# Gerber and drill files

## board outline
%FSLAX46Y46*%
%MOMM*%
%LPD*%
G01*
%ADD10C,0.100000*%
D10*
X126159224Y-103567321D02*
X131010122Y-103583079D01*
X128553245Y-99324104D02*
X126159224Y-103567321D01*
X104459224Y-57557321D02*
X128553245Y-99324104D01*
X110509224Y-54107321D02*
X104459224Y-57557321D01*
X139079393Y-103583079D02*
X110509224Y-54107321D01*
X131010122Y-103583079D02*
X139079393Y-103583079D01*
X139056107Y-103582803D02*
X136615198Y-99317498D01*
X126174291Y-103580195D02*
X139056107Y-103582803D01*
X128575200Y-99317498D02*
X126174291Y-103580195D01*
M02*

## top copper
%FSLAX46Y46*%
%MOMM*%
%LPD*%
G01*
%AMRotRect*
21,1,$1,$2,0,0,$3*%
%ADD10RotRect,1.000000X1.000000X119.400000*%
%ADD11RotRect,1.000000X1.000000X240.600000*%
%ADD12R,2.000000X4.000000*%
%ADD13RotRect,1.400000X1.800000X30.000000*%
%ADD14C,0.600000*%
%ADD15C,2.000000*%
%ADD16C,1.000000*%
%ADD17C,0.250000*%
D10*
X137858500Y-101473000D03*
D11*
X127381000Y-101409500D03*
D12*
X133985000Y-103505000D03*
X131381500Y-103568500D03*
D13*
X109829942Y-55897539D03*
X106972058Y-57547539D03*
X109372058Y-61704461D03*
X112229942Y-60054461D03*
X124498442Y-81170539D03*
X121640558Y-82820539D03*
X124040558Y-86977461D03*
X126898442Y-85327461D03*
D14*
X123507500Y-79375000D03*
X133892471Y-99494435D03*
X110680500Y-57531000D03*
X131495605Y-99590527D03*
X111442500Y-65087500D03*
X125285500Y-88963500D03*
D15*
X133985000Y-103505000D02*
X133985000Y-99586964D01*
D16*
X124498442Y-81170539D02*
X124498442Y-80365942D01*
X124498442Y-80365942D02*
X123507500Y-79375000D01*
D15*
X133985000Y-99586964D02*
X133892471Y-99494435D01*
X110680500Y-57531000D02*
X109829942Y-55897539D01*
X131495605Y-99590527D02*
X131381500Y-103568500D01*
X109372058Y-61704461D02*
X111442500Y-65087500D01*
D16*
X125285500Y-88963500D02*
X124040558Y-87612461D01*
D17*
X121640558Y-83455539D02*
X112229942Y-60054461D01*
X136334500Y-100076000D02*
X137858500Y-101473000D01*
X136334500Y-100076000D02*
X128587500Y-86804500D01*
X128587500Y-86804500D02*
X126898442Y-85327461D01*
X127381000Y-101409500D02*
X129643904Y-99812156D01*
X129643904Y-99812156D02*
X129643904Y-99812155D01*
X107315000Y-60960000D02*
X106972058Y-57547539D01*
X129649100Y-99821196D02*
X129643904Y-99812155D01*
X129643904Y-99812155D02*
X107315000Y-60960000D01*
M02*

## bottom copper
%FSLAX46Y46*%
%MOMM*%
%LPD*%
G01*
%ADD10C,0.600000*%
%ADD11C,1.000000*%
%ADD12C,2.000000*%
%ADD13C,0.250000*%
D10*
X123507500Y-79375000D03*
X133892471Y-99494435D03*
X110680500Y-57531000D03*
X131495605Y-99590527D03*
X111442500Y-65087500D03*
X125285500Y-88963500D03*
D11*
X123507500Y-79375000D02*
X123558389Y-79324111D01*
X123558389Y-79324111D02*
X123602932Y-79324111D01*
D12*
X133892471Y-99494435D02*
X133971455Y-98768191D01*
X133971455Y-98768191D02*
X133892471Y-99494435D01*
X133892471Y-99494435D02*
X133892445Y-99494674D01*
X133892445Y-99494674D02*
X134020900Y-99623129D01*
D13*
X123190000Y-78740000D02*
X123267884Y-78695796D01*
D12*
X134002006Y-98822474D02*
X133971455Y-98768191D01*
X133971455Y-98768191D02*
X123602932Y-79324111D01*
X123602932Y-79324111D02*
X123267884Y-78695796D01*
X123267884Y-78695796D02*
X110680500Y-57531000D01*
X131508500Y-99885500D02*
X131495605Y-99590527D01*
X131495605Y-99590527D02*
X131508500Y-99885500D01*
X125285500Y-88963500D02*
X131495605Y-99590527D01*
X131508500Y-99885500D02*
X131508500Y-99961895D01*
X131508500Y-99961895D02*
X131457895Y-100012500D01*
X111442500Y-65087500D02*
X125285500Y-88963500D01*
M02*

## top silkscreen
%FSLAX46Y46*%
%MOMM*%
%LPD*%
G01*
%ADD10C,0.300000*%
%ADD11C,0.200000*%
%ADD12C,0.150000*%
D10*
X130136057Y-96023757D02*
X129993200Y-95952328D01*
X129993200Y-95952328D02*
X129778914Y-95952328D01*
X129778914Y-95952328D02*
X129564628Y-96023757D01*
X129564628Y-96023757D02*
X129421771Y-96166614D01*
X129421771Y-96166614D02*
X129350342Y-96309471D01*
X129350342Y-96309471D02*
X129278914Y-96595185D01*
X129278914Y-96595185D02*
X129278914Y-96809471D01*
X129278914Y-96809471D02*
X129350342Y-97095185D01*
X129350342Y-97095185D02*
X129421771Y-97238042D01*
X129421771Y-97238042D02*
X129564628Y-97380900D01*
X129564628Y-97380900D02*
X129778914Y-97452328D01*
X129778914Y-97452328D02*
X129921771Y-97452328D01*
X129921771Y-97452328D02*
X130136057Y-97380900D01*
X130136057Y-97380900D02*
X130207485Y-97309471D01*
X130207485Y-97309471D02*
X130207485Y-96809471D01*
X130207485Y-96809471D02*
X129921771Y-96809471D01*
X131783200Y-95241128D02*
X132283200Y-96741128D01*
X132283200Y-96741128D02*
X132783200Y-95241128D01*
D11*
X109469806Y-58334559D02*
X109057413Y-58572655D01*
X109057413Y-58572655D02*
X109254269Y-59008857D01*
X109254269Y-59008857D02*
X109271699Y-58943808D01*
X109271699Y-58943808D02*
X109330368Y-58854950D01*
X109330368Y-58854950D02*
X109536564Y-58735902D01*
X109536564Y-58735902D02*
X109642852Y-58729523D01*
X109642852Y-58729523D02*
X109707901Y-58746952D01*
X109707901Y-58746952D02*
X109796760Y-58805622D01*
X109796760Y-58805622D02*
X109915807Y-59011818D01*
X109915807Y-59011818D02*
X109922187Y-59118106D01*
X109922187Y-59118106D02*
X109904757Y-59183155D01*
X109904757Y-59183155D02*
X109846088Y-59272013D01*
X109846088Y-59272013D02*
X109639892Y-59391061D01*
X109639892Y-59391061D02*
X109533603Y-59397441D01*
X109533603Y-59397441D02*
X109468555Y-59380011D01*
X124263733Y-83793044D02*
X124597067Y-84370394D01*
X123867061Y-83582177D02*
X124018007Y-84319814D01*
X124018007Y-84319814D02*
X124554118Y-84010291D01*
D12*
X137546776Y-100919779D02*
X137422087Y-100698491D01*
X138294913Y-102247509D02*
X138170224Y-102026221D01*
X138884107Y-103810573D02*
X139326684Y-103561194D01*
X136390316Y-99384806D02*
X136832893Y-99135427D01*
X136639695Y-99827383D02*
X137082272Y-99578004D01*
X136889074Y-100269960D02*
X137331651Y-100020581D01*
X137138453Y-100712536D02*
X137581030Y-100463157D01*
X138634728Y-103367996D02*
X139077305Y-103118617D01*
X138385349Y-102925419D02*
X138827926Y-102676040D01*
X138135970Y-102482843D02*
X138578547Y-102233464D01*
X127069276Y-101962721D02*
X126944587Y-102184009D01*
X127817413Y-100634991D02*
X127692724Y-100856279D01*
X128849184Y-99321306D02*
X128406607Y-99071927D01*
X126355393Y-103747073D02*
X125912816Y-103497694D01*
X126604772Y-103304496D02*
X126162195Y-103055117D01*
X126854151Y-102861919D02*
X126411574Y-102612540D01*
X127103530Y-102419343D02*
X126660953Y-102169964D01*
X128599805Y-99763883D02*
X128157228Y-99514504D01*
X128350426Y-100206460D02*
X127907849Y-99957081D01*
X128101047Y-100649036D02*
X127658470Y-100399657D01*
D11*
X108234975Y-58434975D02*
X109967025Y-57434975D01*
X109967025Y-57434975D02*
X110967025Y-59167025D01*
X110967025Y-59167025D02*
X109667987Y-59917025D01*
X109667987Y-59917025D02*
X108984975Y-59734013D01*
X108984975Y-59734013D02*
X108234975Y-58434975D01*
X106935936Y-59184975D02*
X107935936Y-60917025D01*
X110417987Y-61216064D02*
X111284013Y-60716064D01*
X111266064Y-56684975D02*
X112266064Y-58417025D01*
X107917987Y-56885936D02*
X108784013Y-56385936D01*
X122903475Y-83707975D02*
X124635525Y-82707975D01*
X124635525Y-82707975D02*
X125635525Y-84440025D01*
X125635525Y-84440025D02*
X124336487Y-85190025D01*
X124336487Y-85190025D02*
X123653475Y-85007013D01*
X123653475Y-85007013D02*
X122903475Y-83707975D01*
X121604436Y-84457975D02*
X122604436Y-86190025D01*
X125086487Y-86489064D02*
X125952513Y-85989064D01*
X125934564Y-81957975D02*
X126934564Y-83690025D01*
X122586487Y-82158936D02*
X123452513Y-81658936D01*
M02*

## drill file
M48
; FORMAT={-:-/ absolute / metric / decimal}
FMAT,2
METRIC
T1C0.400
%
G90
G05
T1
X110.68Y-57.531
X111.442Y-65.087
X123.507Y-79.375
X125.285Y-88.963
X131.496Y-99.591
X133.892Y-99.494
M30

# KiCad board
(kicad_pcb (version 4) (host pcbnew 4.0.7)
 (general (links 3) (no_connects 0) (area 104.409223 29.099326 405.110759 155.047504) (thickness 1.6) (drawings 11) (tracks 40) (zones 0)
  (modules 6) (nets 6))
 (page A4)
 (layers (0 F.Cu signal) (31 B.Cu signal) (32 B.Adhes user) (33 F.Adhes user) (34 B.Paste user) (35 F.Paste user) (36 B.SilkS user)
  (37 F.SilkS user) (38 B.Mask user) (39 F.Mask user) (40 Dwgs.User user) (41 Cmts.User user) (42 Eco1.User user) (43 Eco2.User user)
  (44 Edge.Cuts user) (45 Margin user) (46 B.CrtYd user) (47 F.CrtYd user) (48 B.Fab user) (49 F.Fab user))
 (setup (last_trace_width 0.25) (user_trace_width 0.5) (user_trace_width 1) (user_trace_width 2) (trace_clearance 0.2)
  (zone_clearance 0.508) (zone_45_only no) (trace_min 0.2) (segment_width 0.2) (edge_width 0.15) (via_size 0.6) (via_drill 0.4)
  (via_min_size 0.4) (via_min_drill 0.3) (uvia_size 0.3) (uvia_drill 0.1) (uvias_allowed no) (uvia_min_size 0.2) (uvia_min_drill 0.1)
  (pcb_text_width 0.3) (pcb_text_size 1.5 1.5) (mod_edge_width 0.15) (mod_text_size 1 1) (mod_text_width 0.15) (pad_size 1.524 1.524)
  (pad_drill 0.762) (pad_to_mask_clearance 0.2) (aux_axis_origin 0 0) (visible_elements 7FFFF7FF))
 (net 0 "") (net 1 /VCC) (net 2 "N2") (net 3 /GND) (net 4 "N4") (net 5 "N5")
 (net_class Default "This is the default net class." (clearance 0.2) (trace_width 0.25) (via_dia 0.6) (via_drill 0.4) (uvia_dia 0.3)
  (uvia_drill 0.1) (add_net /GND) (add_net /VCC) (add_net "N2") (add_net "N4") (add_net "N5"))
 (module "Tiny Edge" (layer F.Cu) (at 137.8585 101.473 119.4)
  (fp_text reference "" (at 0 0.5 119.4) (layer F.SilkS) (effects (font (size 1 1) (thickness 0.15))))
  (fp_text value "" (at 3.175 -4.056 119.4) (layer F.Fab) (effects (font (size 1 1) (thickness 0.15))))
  (fp_line (start 0.635 0) (end 0.889 0) (layer F.SilkS) (width 0.15))
  (fp_line (start -0.889 0) (end -0.635 0) (layer F.SilkS) (width 0.15))
  (fp_line (start -2.54 -0.254) (end -2.54 0.254) (layer F.SilkS) (width 0.15))
  (fp_line (start 2.54 -0.254) (end 2.54 0.254) (layer F.SilkS) (width 0.15))
  (fp_line (start 2.032 -0.254) (end 2.032 0.254) (layer F.SilkS) (width 0.15))
  (fp_line (start 1.524 -0.254) (end 1.524 0.254) (layer F.SilkS) (width 0.15))
  (fp_line (start 1.016 -0.254) (end 1.016 0.254) (layer F.SilkS) (width 0.15))
  (fp_line (start -2.032 -0.254) (end -2.032 0.254) (layer F.SilkS) (width 0.15))
  (fp_line (start -1.524 -0.254) (end -1.524 0.254) (layer F.SilkS) (width 0.15))
  (fp_line (start -1.016 -0.254) (end -1.016 0.254) (layer F.SilkS) (width 0.15))
  (pad 1 smd rect (at 0 0 119.4) (size 1 1) (layers F.Cu F.Paste F.Mask)))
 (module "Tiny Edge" (layer F.Cu) (at 127.381 101.4095 240.6)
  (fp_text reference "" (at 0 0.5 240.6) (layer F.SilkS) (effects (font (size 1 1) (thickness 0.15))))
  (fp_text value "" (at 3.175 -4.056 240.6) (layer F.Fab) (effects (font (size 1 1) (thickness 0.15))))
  (fp_line (start 0.635 0) (end 0.889 0) (layer F.SilkS) (width 0.15))
  (fp_line (start -0.889 0) (end -0.635 0) (layer F.SilkS) (width 0.15))
  (fp_line (start -2.54 -0.254) (end -2.54 0.254) (layer F.SilkS) (width 0.15))
  (fp_line (start 2.54 -0.254) (end 2.54 0.254) (layer F.SilkS) (width 0.15))
  (fp_line (start 2.032 -0.254) (end 2.032 0.254) (layer F.SilkS) (width 0.15))
  (fp_line (start 1.524 -0.254) (end 1.524 0.254) (layer F.SilkS) (width 0.15))
  (fp_line (start 1.016 -0.254) (end 1.016 0.254) (layer F.SilkS) (width 0.15))
  (fp_line (start -2.032 -0.254) (end -2.032 0.254) (layer F.SilkS) (width 0.15))
  (fp_line (start -1.524 -0.254) (end -1.524 0.254) (layer F.SilkS) (width 0.15))
  (fp_line (start -1.016 -0.254) (end -1.016 0.254) (layer F.SilkS) (width 0.15))
  (pad 1 smd rect (at 0 0 240.6) (size 1 1) (layers F.Cu F.Paste F.Mask)))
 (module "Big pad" (layer F.Cu) (at 134.112 103.378 90)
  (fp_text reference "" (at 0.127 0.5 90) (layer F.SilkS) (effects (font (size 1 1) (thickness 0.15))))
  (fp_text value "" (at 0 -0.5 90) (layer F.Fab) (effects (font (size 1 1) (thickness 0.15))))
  (pad 1 smd rect (at -0.127 -0.127 90) (size 4 2) (layers F.Cu F.Paste F.Mask)))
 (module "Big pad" (layer F.Cu) (at 131.5085 103.4415 90)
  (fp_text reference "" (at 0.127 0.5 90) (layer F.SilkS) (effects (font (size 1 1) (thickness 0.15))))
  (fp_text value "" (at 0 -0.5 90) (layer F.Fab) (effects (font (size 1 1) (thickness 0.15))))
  (pad 1 smd rect (at -0.127 -0.127 90) (size 4 2) (layers F.Cu F.Paste F.Mask)))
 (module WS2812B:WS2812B (layer F.Cu) (at 109.601 58.801 30)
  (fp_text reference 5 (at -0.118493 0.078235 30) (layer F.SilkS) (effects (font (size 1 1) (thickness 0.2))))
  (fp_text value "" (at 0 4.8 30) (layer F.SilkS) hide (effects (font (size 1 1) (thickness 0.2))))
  (fp_line (start -1 -1) (end 1 -1) (layer F.SilkS) (width 0.2)) (fp_line (start 1 -1) (end 1 1) (layer F.SilkS) (width 0.2))
  (fp_line (start 1 1) (end -0.5 1) (layer F.SilkS) (width 0.2))
  (fp_line (start -0.5 1) (end -1 0.5) (layer F.SilkS) (width 0.2))
  (fp_line (start -1 0.5) (end -1 -1) (layer F.SilkS) (width 0.2))
  (fp_line (start -2.5 -1) (end -2.5 1) (layer F.SilkS) (width 0.2))
  (fp_line (start -0.5 2.5) (end 0.5 2.5) (layer F.SilkS) (width 0.2))
  (fp_line (start 2.5 -1) (end 2.5 1) (layer F.SilkS) (width 0.2))
  (fp_line (start -0.5 -2.5) (end 0.5 -2.5) (layer F.SilkS) (width 0.2))
  (pad 1 smd rect (at 1.65 -2.4 30) (size 1.4 1.8) (layers F.Cu F.Paste F.Mask) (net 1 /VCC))
  (pad 2 smd rect (at -1.65 -2.4 30) (size 1.4 1.8) (layers F.Cu F.Paste F.Mask) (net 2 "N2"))
  (pad 3 smd rect (at -1.65 2.4 30) (size 1.4 1.8) (layers F.Cu F.Paste F.Mask) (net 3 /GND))
  (pad 4 smd rect (at 1.65 2.4 30) (size 1.4 1.8) (layers F.Cu F.Paste F.Mask) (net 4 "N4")))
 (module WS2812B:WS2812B (layer F.Cu) (at 124.2695 84.074 30)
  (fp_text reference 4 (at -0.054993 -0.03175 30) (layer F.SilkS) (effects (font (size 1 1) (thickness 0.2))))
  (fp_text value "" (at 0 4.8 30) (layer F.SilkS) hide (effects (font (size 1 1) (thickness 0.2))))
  (fp_line (start -1 -1) (end 1 -1) (layer F.SilkS) (width 0.2)) (fp_line (start 1 -1) (end 1 1) (layer F.SilkS) (width 0.2))
  (fp_line (start 1 1) (end -0.5 1) (layer F.SilkS) (width 0.2))
  (fp_line (start -0.5 1) (end -1 0.5) (layer F.SilkS) (width 0.2))
  (fp_line (start -1 0.5) (end -1 -1) (layer F.SilkS) (width 0.2))
  (fp_line (start -2.5 -1) (end -2.5 1) (layer F.SilkS) (width 0.2))
  (fp_line (start -0.5 2.5) (end 0.5 2.5) (layer F.SilkS) (width 0.2))
  (fp_line (start 2.5 -1) (end 2.5 1) (layer F.SilkS) (width 0.2))
  (fp_line (start -0.5 -2.5) (end 0.5 -2.5) (layer F.SilkS) (width 0.2))
  (pad 1 smd rect (at 1.65 -2.4 30) (size 1.4 1.8) (layers F.Cu F.Paste F.Mask) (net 1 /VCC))
  (pad 2 smd rect (at -1.65 -2.4 30) (size 1.4 1.8) (layers F.Cu F.Paste F.Mask) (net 4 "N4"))
  (pad 3 smd rect (at -1.65 2.4 30) (size 1.4 1.8) (layers F.Cu F.Paste F.Mask) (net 3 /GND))
  (pad 4 smd rect (at 1.65 2.4 30) (size 1.4 1.8) (layers F.Cu F.Paste F.Mask) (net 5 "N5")))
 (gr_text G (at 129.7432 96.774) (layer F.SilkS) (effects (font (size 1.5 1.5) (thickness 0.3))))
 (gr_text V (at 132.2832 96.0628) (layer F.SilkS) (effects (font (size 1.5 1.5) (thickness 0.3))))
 (gr_line (start 126.159224 103.567321) (end 131.010122 103.583079) (layer Edge.Cuts) (width 0.1))
 (gr_line (start 128.553245 99.324104) (end 126.159224 103.567321) (layer Edge.Cuts) (width 0.1))
 (gr_line (start 104.459224 57.557321) (end 128.553245 99.324104) (layer Edge.Cuts) (width 0.1))
 (gr_line (start 110.509224 54.107321) (end 104.459224 57.557321) (layer Edge.Cuts) (width 0.1))
 (gr_line (start 139.079393 103.583079) (end 110.509224 54.107321) (layer Edge.Cuts) (width 0.1))
 (gr_line (start 131.010122 103.583079) (end 139.079393 103.583079) (layer Edge.Cuts) (width 0.1))
 (gr_line (start 139.056107 103.582803) (end 136.615198 99.317498) (layer Edge.Cuts) (width 0.1))
 (gr_line (start 126.174291 103.580195) (end 139.056107 103.582803) (layer Edge.Cuts) (width 0.1))
 (gr_line (start 128.5752 99.317498) (end 126.174291 103.580195) (layer Edge.Cuts) (width 0.1))
 (segment (start 133.985 103.505) (end 133.985 99.586964) (width 2) (layer F.Cu) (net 1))
 (segment (start 124.498442 81.170539) (end 124.498442 80.365942) (width 1) (layer F.Cu) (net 1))
 (segment (start 124.498442 80.365942) (end 123.5075 79.375) (width 1) (layer F.Cu) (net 1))
 (via (at 123.5075 79.375) (size 0.6) (drill 0.4) (layers F.Cu B.Cu) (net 1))
 (segment (start 123.5075 79.375) (end 123.558389 79.324111) (width 1) (layer B.Cu) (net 1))
 (segment (start 123.558389 79.324111) (end 123.602932 79.324111) (width 1) (layer B.Cu) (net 1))
 (via (at 133.892471 99.494435) (size 0.6) (drill 0.4) (layers F.Cu B.Cu) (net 1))
 (segment (start 133.985 99.586964) (end 133.892471 99.494435) (width 2) (layer F.Cu) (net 1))
 (segment (start 133.892471 99.494435) (end 133.971455 98.768191) (width 2) (layer B.Cu) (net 1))
 (segment (start 133.971455 98.768191) (end 133.892471 99.494435) (width 2) (layer B.Cu) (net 1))
 (segment (start 133.892471 99.494435) (end 133.892445 99.494674) (width 2) (layer B.Cu) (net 1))
 (segment (start 133.892445 99.494674) (end 134.0209 99.623129) (width 2) (layer B.Cu) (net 1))
 (segment (start 123.19 78.74) (end 123.267884 78.695796) (width 0.25) (layer B.Cu) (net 1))
 (segment (start 134.002006 98.822474) (end 133.971455 98.768191) (width 2) (layer B.Cu) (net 1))
 (segment (start 133.971455 98.768191) (end 123.602932 79.324111) (width 2) (layer B.Cu) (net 1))
 (segment (start 123.602932 79.324111) (end 123.267884 78.695796) (width 2) (layer B.Cu) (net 1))
 (segment (start 123.267884 78.695796) (end 110.6805 57.531) (width 2) (layer B.Cu) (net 1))
 (via (at 110.6805 57.531) (size 0.6) (drill 0.4) (layers F.Cu B.Cu) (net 1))
 (segment (start 110.6805 57.531) (end 109.829942 55.897539) (width 2) (layer F.Cu) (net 1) (status 20))
 (segment (start 131.5085 99.8855) (end 131.495605 99.590527) (width 2) (layer B.Cu) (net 3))
 (via (at 131.495605 99.590527) (size 0.6) (drill 0.4) (layers F.Cu B.Cu) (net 3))
 (segment (start 131.495605 99.590527) (end 131.3815 103.5685) (width 2) (layer F.Cu) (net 3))
 (segment (start 131.495605 99.590527) (end 131.5085 99.8855) (width 2) (layer B.Cu) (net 3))
 (segment (start 125.2855 88.9635) (end 131.495605 99.590527) (width 2) (layer B.Cu) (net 3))
 (segment (start 131.5085 99.8855) (end 131.5085 99.961895) (width 2) (layer B.Cu) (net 3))
 (segment (start 131.5085 99.961895) (end 131.457895 100.0125) (width 2) (layer B.Cu) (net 3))
 (segment (start 109.372058 61.704461) (end 111.4425 65.0875) (width 2) (layer F.Cu) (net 3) (status 10))
 (segment (start 111.4425 65.0875) (end 125.2855 88.9635) (width 2) (layer B.Cu) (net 3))
 (via (at 111.4425 65.0875) (size 0.6) (drill 0.4) (layers F.Cu B.Cu) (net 3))
 (segment (start 125.2855 88.9635) (end 124.040558 87.612461) (width 1) (layer F.Cu) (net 3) (status 20))
 (via (at 125.2855 88.9635) (size 0.6) (drill 0.4) (layers F.Cu B.Cu) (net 3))
 (segment (start 121.640558 83.455539) (end 112.229942 60.054461) (width 0.25) (layer F.Cu) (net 4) (status 10))
 (segment (start 136.3345 100.076) (end 137.8585 101.473) (width 0.25) (layer F.Cu) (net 5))
 (segment (start 136.3345 100.076) (end 128.5875 86.8045) (width 0.25) (layer F.Cu) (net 5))
 (segment (start 128.5875 86.8045) (end 126.898442 85.327461) (width 0.25) (layer F.Cu) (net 5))
 (segment (start 127.381 101.4095) (end 129.643904 99.812156) (width 0.25) (layer F.Cu) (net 2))
 (segment (start 129.643904 99.812156) (end 129.643904 99.812155) (width 0.25) (layer F.Cu) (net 2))
 (segment (start 107.315 60.96) (end 106.972058 57.547539) (width 0.25) (layer F.Cu) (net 2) (status 20))
 (segment (start 129.6491 99.821196) (end 129.643904 99.812155) (width 0.25) (layer F.Cu) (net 2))
 (segment (start 129.643904 99.812155) (end 107.315 60.96) (width 0.25) (layer F.Cu) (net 2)))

